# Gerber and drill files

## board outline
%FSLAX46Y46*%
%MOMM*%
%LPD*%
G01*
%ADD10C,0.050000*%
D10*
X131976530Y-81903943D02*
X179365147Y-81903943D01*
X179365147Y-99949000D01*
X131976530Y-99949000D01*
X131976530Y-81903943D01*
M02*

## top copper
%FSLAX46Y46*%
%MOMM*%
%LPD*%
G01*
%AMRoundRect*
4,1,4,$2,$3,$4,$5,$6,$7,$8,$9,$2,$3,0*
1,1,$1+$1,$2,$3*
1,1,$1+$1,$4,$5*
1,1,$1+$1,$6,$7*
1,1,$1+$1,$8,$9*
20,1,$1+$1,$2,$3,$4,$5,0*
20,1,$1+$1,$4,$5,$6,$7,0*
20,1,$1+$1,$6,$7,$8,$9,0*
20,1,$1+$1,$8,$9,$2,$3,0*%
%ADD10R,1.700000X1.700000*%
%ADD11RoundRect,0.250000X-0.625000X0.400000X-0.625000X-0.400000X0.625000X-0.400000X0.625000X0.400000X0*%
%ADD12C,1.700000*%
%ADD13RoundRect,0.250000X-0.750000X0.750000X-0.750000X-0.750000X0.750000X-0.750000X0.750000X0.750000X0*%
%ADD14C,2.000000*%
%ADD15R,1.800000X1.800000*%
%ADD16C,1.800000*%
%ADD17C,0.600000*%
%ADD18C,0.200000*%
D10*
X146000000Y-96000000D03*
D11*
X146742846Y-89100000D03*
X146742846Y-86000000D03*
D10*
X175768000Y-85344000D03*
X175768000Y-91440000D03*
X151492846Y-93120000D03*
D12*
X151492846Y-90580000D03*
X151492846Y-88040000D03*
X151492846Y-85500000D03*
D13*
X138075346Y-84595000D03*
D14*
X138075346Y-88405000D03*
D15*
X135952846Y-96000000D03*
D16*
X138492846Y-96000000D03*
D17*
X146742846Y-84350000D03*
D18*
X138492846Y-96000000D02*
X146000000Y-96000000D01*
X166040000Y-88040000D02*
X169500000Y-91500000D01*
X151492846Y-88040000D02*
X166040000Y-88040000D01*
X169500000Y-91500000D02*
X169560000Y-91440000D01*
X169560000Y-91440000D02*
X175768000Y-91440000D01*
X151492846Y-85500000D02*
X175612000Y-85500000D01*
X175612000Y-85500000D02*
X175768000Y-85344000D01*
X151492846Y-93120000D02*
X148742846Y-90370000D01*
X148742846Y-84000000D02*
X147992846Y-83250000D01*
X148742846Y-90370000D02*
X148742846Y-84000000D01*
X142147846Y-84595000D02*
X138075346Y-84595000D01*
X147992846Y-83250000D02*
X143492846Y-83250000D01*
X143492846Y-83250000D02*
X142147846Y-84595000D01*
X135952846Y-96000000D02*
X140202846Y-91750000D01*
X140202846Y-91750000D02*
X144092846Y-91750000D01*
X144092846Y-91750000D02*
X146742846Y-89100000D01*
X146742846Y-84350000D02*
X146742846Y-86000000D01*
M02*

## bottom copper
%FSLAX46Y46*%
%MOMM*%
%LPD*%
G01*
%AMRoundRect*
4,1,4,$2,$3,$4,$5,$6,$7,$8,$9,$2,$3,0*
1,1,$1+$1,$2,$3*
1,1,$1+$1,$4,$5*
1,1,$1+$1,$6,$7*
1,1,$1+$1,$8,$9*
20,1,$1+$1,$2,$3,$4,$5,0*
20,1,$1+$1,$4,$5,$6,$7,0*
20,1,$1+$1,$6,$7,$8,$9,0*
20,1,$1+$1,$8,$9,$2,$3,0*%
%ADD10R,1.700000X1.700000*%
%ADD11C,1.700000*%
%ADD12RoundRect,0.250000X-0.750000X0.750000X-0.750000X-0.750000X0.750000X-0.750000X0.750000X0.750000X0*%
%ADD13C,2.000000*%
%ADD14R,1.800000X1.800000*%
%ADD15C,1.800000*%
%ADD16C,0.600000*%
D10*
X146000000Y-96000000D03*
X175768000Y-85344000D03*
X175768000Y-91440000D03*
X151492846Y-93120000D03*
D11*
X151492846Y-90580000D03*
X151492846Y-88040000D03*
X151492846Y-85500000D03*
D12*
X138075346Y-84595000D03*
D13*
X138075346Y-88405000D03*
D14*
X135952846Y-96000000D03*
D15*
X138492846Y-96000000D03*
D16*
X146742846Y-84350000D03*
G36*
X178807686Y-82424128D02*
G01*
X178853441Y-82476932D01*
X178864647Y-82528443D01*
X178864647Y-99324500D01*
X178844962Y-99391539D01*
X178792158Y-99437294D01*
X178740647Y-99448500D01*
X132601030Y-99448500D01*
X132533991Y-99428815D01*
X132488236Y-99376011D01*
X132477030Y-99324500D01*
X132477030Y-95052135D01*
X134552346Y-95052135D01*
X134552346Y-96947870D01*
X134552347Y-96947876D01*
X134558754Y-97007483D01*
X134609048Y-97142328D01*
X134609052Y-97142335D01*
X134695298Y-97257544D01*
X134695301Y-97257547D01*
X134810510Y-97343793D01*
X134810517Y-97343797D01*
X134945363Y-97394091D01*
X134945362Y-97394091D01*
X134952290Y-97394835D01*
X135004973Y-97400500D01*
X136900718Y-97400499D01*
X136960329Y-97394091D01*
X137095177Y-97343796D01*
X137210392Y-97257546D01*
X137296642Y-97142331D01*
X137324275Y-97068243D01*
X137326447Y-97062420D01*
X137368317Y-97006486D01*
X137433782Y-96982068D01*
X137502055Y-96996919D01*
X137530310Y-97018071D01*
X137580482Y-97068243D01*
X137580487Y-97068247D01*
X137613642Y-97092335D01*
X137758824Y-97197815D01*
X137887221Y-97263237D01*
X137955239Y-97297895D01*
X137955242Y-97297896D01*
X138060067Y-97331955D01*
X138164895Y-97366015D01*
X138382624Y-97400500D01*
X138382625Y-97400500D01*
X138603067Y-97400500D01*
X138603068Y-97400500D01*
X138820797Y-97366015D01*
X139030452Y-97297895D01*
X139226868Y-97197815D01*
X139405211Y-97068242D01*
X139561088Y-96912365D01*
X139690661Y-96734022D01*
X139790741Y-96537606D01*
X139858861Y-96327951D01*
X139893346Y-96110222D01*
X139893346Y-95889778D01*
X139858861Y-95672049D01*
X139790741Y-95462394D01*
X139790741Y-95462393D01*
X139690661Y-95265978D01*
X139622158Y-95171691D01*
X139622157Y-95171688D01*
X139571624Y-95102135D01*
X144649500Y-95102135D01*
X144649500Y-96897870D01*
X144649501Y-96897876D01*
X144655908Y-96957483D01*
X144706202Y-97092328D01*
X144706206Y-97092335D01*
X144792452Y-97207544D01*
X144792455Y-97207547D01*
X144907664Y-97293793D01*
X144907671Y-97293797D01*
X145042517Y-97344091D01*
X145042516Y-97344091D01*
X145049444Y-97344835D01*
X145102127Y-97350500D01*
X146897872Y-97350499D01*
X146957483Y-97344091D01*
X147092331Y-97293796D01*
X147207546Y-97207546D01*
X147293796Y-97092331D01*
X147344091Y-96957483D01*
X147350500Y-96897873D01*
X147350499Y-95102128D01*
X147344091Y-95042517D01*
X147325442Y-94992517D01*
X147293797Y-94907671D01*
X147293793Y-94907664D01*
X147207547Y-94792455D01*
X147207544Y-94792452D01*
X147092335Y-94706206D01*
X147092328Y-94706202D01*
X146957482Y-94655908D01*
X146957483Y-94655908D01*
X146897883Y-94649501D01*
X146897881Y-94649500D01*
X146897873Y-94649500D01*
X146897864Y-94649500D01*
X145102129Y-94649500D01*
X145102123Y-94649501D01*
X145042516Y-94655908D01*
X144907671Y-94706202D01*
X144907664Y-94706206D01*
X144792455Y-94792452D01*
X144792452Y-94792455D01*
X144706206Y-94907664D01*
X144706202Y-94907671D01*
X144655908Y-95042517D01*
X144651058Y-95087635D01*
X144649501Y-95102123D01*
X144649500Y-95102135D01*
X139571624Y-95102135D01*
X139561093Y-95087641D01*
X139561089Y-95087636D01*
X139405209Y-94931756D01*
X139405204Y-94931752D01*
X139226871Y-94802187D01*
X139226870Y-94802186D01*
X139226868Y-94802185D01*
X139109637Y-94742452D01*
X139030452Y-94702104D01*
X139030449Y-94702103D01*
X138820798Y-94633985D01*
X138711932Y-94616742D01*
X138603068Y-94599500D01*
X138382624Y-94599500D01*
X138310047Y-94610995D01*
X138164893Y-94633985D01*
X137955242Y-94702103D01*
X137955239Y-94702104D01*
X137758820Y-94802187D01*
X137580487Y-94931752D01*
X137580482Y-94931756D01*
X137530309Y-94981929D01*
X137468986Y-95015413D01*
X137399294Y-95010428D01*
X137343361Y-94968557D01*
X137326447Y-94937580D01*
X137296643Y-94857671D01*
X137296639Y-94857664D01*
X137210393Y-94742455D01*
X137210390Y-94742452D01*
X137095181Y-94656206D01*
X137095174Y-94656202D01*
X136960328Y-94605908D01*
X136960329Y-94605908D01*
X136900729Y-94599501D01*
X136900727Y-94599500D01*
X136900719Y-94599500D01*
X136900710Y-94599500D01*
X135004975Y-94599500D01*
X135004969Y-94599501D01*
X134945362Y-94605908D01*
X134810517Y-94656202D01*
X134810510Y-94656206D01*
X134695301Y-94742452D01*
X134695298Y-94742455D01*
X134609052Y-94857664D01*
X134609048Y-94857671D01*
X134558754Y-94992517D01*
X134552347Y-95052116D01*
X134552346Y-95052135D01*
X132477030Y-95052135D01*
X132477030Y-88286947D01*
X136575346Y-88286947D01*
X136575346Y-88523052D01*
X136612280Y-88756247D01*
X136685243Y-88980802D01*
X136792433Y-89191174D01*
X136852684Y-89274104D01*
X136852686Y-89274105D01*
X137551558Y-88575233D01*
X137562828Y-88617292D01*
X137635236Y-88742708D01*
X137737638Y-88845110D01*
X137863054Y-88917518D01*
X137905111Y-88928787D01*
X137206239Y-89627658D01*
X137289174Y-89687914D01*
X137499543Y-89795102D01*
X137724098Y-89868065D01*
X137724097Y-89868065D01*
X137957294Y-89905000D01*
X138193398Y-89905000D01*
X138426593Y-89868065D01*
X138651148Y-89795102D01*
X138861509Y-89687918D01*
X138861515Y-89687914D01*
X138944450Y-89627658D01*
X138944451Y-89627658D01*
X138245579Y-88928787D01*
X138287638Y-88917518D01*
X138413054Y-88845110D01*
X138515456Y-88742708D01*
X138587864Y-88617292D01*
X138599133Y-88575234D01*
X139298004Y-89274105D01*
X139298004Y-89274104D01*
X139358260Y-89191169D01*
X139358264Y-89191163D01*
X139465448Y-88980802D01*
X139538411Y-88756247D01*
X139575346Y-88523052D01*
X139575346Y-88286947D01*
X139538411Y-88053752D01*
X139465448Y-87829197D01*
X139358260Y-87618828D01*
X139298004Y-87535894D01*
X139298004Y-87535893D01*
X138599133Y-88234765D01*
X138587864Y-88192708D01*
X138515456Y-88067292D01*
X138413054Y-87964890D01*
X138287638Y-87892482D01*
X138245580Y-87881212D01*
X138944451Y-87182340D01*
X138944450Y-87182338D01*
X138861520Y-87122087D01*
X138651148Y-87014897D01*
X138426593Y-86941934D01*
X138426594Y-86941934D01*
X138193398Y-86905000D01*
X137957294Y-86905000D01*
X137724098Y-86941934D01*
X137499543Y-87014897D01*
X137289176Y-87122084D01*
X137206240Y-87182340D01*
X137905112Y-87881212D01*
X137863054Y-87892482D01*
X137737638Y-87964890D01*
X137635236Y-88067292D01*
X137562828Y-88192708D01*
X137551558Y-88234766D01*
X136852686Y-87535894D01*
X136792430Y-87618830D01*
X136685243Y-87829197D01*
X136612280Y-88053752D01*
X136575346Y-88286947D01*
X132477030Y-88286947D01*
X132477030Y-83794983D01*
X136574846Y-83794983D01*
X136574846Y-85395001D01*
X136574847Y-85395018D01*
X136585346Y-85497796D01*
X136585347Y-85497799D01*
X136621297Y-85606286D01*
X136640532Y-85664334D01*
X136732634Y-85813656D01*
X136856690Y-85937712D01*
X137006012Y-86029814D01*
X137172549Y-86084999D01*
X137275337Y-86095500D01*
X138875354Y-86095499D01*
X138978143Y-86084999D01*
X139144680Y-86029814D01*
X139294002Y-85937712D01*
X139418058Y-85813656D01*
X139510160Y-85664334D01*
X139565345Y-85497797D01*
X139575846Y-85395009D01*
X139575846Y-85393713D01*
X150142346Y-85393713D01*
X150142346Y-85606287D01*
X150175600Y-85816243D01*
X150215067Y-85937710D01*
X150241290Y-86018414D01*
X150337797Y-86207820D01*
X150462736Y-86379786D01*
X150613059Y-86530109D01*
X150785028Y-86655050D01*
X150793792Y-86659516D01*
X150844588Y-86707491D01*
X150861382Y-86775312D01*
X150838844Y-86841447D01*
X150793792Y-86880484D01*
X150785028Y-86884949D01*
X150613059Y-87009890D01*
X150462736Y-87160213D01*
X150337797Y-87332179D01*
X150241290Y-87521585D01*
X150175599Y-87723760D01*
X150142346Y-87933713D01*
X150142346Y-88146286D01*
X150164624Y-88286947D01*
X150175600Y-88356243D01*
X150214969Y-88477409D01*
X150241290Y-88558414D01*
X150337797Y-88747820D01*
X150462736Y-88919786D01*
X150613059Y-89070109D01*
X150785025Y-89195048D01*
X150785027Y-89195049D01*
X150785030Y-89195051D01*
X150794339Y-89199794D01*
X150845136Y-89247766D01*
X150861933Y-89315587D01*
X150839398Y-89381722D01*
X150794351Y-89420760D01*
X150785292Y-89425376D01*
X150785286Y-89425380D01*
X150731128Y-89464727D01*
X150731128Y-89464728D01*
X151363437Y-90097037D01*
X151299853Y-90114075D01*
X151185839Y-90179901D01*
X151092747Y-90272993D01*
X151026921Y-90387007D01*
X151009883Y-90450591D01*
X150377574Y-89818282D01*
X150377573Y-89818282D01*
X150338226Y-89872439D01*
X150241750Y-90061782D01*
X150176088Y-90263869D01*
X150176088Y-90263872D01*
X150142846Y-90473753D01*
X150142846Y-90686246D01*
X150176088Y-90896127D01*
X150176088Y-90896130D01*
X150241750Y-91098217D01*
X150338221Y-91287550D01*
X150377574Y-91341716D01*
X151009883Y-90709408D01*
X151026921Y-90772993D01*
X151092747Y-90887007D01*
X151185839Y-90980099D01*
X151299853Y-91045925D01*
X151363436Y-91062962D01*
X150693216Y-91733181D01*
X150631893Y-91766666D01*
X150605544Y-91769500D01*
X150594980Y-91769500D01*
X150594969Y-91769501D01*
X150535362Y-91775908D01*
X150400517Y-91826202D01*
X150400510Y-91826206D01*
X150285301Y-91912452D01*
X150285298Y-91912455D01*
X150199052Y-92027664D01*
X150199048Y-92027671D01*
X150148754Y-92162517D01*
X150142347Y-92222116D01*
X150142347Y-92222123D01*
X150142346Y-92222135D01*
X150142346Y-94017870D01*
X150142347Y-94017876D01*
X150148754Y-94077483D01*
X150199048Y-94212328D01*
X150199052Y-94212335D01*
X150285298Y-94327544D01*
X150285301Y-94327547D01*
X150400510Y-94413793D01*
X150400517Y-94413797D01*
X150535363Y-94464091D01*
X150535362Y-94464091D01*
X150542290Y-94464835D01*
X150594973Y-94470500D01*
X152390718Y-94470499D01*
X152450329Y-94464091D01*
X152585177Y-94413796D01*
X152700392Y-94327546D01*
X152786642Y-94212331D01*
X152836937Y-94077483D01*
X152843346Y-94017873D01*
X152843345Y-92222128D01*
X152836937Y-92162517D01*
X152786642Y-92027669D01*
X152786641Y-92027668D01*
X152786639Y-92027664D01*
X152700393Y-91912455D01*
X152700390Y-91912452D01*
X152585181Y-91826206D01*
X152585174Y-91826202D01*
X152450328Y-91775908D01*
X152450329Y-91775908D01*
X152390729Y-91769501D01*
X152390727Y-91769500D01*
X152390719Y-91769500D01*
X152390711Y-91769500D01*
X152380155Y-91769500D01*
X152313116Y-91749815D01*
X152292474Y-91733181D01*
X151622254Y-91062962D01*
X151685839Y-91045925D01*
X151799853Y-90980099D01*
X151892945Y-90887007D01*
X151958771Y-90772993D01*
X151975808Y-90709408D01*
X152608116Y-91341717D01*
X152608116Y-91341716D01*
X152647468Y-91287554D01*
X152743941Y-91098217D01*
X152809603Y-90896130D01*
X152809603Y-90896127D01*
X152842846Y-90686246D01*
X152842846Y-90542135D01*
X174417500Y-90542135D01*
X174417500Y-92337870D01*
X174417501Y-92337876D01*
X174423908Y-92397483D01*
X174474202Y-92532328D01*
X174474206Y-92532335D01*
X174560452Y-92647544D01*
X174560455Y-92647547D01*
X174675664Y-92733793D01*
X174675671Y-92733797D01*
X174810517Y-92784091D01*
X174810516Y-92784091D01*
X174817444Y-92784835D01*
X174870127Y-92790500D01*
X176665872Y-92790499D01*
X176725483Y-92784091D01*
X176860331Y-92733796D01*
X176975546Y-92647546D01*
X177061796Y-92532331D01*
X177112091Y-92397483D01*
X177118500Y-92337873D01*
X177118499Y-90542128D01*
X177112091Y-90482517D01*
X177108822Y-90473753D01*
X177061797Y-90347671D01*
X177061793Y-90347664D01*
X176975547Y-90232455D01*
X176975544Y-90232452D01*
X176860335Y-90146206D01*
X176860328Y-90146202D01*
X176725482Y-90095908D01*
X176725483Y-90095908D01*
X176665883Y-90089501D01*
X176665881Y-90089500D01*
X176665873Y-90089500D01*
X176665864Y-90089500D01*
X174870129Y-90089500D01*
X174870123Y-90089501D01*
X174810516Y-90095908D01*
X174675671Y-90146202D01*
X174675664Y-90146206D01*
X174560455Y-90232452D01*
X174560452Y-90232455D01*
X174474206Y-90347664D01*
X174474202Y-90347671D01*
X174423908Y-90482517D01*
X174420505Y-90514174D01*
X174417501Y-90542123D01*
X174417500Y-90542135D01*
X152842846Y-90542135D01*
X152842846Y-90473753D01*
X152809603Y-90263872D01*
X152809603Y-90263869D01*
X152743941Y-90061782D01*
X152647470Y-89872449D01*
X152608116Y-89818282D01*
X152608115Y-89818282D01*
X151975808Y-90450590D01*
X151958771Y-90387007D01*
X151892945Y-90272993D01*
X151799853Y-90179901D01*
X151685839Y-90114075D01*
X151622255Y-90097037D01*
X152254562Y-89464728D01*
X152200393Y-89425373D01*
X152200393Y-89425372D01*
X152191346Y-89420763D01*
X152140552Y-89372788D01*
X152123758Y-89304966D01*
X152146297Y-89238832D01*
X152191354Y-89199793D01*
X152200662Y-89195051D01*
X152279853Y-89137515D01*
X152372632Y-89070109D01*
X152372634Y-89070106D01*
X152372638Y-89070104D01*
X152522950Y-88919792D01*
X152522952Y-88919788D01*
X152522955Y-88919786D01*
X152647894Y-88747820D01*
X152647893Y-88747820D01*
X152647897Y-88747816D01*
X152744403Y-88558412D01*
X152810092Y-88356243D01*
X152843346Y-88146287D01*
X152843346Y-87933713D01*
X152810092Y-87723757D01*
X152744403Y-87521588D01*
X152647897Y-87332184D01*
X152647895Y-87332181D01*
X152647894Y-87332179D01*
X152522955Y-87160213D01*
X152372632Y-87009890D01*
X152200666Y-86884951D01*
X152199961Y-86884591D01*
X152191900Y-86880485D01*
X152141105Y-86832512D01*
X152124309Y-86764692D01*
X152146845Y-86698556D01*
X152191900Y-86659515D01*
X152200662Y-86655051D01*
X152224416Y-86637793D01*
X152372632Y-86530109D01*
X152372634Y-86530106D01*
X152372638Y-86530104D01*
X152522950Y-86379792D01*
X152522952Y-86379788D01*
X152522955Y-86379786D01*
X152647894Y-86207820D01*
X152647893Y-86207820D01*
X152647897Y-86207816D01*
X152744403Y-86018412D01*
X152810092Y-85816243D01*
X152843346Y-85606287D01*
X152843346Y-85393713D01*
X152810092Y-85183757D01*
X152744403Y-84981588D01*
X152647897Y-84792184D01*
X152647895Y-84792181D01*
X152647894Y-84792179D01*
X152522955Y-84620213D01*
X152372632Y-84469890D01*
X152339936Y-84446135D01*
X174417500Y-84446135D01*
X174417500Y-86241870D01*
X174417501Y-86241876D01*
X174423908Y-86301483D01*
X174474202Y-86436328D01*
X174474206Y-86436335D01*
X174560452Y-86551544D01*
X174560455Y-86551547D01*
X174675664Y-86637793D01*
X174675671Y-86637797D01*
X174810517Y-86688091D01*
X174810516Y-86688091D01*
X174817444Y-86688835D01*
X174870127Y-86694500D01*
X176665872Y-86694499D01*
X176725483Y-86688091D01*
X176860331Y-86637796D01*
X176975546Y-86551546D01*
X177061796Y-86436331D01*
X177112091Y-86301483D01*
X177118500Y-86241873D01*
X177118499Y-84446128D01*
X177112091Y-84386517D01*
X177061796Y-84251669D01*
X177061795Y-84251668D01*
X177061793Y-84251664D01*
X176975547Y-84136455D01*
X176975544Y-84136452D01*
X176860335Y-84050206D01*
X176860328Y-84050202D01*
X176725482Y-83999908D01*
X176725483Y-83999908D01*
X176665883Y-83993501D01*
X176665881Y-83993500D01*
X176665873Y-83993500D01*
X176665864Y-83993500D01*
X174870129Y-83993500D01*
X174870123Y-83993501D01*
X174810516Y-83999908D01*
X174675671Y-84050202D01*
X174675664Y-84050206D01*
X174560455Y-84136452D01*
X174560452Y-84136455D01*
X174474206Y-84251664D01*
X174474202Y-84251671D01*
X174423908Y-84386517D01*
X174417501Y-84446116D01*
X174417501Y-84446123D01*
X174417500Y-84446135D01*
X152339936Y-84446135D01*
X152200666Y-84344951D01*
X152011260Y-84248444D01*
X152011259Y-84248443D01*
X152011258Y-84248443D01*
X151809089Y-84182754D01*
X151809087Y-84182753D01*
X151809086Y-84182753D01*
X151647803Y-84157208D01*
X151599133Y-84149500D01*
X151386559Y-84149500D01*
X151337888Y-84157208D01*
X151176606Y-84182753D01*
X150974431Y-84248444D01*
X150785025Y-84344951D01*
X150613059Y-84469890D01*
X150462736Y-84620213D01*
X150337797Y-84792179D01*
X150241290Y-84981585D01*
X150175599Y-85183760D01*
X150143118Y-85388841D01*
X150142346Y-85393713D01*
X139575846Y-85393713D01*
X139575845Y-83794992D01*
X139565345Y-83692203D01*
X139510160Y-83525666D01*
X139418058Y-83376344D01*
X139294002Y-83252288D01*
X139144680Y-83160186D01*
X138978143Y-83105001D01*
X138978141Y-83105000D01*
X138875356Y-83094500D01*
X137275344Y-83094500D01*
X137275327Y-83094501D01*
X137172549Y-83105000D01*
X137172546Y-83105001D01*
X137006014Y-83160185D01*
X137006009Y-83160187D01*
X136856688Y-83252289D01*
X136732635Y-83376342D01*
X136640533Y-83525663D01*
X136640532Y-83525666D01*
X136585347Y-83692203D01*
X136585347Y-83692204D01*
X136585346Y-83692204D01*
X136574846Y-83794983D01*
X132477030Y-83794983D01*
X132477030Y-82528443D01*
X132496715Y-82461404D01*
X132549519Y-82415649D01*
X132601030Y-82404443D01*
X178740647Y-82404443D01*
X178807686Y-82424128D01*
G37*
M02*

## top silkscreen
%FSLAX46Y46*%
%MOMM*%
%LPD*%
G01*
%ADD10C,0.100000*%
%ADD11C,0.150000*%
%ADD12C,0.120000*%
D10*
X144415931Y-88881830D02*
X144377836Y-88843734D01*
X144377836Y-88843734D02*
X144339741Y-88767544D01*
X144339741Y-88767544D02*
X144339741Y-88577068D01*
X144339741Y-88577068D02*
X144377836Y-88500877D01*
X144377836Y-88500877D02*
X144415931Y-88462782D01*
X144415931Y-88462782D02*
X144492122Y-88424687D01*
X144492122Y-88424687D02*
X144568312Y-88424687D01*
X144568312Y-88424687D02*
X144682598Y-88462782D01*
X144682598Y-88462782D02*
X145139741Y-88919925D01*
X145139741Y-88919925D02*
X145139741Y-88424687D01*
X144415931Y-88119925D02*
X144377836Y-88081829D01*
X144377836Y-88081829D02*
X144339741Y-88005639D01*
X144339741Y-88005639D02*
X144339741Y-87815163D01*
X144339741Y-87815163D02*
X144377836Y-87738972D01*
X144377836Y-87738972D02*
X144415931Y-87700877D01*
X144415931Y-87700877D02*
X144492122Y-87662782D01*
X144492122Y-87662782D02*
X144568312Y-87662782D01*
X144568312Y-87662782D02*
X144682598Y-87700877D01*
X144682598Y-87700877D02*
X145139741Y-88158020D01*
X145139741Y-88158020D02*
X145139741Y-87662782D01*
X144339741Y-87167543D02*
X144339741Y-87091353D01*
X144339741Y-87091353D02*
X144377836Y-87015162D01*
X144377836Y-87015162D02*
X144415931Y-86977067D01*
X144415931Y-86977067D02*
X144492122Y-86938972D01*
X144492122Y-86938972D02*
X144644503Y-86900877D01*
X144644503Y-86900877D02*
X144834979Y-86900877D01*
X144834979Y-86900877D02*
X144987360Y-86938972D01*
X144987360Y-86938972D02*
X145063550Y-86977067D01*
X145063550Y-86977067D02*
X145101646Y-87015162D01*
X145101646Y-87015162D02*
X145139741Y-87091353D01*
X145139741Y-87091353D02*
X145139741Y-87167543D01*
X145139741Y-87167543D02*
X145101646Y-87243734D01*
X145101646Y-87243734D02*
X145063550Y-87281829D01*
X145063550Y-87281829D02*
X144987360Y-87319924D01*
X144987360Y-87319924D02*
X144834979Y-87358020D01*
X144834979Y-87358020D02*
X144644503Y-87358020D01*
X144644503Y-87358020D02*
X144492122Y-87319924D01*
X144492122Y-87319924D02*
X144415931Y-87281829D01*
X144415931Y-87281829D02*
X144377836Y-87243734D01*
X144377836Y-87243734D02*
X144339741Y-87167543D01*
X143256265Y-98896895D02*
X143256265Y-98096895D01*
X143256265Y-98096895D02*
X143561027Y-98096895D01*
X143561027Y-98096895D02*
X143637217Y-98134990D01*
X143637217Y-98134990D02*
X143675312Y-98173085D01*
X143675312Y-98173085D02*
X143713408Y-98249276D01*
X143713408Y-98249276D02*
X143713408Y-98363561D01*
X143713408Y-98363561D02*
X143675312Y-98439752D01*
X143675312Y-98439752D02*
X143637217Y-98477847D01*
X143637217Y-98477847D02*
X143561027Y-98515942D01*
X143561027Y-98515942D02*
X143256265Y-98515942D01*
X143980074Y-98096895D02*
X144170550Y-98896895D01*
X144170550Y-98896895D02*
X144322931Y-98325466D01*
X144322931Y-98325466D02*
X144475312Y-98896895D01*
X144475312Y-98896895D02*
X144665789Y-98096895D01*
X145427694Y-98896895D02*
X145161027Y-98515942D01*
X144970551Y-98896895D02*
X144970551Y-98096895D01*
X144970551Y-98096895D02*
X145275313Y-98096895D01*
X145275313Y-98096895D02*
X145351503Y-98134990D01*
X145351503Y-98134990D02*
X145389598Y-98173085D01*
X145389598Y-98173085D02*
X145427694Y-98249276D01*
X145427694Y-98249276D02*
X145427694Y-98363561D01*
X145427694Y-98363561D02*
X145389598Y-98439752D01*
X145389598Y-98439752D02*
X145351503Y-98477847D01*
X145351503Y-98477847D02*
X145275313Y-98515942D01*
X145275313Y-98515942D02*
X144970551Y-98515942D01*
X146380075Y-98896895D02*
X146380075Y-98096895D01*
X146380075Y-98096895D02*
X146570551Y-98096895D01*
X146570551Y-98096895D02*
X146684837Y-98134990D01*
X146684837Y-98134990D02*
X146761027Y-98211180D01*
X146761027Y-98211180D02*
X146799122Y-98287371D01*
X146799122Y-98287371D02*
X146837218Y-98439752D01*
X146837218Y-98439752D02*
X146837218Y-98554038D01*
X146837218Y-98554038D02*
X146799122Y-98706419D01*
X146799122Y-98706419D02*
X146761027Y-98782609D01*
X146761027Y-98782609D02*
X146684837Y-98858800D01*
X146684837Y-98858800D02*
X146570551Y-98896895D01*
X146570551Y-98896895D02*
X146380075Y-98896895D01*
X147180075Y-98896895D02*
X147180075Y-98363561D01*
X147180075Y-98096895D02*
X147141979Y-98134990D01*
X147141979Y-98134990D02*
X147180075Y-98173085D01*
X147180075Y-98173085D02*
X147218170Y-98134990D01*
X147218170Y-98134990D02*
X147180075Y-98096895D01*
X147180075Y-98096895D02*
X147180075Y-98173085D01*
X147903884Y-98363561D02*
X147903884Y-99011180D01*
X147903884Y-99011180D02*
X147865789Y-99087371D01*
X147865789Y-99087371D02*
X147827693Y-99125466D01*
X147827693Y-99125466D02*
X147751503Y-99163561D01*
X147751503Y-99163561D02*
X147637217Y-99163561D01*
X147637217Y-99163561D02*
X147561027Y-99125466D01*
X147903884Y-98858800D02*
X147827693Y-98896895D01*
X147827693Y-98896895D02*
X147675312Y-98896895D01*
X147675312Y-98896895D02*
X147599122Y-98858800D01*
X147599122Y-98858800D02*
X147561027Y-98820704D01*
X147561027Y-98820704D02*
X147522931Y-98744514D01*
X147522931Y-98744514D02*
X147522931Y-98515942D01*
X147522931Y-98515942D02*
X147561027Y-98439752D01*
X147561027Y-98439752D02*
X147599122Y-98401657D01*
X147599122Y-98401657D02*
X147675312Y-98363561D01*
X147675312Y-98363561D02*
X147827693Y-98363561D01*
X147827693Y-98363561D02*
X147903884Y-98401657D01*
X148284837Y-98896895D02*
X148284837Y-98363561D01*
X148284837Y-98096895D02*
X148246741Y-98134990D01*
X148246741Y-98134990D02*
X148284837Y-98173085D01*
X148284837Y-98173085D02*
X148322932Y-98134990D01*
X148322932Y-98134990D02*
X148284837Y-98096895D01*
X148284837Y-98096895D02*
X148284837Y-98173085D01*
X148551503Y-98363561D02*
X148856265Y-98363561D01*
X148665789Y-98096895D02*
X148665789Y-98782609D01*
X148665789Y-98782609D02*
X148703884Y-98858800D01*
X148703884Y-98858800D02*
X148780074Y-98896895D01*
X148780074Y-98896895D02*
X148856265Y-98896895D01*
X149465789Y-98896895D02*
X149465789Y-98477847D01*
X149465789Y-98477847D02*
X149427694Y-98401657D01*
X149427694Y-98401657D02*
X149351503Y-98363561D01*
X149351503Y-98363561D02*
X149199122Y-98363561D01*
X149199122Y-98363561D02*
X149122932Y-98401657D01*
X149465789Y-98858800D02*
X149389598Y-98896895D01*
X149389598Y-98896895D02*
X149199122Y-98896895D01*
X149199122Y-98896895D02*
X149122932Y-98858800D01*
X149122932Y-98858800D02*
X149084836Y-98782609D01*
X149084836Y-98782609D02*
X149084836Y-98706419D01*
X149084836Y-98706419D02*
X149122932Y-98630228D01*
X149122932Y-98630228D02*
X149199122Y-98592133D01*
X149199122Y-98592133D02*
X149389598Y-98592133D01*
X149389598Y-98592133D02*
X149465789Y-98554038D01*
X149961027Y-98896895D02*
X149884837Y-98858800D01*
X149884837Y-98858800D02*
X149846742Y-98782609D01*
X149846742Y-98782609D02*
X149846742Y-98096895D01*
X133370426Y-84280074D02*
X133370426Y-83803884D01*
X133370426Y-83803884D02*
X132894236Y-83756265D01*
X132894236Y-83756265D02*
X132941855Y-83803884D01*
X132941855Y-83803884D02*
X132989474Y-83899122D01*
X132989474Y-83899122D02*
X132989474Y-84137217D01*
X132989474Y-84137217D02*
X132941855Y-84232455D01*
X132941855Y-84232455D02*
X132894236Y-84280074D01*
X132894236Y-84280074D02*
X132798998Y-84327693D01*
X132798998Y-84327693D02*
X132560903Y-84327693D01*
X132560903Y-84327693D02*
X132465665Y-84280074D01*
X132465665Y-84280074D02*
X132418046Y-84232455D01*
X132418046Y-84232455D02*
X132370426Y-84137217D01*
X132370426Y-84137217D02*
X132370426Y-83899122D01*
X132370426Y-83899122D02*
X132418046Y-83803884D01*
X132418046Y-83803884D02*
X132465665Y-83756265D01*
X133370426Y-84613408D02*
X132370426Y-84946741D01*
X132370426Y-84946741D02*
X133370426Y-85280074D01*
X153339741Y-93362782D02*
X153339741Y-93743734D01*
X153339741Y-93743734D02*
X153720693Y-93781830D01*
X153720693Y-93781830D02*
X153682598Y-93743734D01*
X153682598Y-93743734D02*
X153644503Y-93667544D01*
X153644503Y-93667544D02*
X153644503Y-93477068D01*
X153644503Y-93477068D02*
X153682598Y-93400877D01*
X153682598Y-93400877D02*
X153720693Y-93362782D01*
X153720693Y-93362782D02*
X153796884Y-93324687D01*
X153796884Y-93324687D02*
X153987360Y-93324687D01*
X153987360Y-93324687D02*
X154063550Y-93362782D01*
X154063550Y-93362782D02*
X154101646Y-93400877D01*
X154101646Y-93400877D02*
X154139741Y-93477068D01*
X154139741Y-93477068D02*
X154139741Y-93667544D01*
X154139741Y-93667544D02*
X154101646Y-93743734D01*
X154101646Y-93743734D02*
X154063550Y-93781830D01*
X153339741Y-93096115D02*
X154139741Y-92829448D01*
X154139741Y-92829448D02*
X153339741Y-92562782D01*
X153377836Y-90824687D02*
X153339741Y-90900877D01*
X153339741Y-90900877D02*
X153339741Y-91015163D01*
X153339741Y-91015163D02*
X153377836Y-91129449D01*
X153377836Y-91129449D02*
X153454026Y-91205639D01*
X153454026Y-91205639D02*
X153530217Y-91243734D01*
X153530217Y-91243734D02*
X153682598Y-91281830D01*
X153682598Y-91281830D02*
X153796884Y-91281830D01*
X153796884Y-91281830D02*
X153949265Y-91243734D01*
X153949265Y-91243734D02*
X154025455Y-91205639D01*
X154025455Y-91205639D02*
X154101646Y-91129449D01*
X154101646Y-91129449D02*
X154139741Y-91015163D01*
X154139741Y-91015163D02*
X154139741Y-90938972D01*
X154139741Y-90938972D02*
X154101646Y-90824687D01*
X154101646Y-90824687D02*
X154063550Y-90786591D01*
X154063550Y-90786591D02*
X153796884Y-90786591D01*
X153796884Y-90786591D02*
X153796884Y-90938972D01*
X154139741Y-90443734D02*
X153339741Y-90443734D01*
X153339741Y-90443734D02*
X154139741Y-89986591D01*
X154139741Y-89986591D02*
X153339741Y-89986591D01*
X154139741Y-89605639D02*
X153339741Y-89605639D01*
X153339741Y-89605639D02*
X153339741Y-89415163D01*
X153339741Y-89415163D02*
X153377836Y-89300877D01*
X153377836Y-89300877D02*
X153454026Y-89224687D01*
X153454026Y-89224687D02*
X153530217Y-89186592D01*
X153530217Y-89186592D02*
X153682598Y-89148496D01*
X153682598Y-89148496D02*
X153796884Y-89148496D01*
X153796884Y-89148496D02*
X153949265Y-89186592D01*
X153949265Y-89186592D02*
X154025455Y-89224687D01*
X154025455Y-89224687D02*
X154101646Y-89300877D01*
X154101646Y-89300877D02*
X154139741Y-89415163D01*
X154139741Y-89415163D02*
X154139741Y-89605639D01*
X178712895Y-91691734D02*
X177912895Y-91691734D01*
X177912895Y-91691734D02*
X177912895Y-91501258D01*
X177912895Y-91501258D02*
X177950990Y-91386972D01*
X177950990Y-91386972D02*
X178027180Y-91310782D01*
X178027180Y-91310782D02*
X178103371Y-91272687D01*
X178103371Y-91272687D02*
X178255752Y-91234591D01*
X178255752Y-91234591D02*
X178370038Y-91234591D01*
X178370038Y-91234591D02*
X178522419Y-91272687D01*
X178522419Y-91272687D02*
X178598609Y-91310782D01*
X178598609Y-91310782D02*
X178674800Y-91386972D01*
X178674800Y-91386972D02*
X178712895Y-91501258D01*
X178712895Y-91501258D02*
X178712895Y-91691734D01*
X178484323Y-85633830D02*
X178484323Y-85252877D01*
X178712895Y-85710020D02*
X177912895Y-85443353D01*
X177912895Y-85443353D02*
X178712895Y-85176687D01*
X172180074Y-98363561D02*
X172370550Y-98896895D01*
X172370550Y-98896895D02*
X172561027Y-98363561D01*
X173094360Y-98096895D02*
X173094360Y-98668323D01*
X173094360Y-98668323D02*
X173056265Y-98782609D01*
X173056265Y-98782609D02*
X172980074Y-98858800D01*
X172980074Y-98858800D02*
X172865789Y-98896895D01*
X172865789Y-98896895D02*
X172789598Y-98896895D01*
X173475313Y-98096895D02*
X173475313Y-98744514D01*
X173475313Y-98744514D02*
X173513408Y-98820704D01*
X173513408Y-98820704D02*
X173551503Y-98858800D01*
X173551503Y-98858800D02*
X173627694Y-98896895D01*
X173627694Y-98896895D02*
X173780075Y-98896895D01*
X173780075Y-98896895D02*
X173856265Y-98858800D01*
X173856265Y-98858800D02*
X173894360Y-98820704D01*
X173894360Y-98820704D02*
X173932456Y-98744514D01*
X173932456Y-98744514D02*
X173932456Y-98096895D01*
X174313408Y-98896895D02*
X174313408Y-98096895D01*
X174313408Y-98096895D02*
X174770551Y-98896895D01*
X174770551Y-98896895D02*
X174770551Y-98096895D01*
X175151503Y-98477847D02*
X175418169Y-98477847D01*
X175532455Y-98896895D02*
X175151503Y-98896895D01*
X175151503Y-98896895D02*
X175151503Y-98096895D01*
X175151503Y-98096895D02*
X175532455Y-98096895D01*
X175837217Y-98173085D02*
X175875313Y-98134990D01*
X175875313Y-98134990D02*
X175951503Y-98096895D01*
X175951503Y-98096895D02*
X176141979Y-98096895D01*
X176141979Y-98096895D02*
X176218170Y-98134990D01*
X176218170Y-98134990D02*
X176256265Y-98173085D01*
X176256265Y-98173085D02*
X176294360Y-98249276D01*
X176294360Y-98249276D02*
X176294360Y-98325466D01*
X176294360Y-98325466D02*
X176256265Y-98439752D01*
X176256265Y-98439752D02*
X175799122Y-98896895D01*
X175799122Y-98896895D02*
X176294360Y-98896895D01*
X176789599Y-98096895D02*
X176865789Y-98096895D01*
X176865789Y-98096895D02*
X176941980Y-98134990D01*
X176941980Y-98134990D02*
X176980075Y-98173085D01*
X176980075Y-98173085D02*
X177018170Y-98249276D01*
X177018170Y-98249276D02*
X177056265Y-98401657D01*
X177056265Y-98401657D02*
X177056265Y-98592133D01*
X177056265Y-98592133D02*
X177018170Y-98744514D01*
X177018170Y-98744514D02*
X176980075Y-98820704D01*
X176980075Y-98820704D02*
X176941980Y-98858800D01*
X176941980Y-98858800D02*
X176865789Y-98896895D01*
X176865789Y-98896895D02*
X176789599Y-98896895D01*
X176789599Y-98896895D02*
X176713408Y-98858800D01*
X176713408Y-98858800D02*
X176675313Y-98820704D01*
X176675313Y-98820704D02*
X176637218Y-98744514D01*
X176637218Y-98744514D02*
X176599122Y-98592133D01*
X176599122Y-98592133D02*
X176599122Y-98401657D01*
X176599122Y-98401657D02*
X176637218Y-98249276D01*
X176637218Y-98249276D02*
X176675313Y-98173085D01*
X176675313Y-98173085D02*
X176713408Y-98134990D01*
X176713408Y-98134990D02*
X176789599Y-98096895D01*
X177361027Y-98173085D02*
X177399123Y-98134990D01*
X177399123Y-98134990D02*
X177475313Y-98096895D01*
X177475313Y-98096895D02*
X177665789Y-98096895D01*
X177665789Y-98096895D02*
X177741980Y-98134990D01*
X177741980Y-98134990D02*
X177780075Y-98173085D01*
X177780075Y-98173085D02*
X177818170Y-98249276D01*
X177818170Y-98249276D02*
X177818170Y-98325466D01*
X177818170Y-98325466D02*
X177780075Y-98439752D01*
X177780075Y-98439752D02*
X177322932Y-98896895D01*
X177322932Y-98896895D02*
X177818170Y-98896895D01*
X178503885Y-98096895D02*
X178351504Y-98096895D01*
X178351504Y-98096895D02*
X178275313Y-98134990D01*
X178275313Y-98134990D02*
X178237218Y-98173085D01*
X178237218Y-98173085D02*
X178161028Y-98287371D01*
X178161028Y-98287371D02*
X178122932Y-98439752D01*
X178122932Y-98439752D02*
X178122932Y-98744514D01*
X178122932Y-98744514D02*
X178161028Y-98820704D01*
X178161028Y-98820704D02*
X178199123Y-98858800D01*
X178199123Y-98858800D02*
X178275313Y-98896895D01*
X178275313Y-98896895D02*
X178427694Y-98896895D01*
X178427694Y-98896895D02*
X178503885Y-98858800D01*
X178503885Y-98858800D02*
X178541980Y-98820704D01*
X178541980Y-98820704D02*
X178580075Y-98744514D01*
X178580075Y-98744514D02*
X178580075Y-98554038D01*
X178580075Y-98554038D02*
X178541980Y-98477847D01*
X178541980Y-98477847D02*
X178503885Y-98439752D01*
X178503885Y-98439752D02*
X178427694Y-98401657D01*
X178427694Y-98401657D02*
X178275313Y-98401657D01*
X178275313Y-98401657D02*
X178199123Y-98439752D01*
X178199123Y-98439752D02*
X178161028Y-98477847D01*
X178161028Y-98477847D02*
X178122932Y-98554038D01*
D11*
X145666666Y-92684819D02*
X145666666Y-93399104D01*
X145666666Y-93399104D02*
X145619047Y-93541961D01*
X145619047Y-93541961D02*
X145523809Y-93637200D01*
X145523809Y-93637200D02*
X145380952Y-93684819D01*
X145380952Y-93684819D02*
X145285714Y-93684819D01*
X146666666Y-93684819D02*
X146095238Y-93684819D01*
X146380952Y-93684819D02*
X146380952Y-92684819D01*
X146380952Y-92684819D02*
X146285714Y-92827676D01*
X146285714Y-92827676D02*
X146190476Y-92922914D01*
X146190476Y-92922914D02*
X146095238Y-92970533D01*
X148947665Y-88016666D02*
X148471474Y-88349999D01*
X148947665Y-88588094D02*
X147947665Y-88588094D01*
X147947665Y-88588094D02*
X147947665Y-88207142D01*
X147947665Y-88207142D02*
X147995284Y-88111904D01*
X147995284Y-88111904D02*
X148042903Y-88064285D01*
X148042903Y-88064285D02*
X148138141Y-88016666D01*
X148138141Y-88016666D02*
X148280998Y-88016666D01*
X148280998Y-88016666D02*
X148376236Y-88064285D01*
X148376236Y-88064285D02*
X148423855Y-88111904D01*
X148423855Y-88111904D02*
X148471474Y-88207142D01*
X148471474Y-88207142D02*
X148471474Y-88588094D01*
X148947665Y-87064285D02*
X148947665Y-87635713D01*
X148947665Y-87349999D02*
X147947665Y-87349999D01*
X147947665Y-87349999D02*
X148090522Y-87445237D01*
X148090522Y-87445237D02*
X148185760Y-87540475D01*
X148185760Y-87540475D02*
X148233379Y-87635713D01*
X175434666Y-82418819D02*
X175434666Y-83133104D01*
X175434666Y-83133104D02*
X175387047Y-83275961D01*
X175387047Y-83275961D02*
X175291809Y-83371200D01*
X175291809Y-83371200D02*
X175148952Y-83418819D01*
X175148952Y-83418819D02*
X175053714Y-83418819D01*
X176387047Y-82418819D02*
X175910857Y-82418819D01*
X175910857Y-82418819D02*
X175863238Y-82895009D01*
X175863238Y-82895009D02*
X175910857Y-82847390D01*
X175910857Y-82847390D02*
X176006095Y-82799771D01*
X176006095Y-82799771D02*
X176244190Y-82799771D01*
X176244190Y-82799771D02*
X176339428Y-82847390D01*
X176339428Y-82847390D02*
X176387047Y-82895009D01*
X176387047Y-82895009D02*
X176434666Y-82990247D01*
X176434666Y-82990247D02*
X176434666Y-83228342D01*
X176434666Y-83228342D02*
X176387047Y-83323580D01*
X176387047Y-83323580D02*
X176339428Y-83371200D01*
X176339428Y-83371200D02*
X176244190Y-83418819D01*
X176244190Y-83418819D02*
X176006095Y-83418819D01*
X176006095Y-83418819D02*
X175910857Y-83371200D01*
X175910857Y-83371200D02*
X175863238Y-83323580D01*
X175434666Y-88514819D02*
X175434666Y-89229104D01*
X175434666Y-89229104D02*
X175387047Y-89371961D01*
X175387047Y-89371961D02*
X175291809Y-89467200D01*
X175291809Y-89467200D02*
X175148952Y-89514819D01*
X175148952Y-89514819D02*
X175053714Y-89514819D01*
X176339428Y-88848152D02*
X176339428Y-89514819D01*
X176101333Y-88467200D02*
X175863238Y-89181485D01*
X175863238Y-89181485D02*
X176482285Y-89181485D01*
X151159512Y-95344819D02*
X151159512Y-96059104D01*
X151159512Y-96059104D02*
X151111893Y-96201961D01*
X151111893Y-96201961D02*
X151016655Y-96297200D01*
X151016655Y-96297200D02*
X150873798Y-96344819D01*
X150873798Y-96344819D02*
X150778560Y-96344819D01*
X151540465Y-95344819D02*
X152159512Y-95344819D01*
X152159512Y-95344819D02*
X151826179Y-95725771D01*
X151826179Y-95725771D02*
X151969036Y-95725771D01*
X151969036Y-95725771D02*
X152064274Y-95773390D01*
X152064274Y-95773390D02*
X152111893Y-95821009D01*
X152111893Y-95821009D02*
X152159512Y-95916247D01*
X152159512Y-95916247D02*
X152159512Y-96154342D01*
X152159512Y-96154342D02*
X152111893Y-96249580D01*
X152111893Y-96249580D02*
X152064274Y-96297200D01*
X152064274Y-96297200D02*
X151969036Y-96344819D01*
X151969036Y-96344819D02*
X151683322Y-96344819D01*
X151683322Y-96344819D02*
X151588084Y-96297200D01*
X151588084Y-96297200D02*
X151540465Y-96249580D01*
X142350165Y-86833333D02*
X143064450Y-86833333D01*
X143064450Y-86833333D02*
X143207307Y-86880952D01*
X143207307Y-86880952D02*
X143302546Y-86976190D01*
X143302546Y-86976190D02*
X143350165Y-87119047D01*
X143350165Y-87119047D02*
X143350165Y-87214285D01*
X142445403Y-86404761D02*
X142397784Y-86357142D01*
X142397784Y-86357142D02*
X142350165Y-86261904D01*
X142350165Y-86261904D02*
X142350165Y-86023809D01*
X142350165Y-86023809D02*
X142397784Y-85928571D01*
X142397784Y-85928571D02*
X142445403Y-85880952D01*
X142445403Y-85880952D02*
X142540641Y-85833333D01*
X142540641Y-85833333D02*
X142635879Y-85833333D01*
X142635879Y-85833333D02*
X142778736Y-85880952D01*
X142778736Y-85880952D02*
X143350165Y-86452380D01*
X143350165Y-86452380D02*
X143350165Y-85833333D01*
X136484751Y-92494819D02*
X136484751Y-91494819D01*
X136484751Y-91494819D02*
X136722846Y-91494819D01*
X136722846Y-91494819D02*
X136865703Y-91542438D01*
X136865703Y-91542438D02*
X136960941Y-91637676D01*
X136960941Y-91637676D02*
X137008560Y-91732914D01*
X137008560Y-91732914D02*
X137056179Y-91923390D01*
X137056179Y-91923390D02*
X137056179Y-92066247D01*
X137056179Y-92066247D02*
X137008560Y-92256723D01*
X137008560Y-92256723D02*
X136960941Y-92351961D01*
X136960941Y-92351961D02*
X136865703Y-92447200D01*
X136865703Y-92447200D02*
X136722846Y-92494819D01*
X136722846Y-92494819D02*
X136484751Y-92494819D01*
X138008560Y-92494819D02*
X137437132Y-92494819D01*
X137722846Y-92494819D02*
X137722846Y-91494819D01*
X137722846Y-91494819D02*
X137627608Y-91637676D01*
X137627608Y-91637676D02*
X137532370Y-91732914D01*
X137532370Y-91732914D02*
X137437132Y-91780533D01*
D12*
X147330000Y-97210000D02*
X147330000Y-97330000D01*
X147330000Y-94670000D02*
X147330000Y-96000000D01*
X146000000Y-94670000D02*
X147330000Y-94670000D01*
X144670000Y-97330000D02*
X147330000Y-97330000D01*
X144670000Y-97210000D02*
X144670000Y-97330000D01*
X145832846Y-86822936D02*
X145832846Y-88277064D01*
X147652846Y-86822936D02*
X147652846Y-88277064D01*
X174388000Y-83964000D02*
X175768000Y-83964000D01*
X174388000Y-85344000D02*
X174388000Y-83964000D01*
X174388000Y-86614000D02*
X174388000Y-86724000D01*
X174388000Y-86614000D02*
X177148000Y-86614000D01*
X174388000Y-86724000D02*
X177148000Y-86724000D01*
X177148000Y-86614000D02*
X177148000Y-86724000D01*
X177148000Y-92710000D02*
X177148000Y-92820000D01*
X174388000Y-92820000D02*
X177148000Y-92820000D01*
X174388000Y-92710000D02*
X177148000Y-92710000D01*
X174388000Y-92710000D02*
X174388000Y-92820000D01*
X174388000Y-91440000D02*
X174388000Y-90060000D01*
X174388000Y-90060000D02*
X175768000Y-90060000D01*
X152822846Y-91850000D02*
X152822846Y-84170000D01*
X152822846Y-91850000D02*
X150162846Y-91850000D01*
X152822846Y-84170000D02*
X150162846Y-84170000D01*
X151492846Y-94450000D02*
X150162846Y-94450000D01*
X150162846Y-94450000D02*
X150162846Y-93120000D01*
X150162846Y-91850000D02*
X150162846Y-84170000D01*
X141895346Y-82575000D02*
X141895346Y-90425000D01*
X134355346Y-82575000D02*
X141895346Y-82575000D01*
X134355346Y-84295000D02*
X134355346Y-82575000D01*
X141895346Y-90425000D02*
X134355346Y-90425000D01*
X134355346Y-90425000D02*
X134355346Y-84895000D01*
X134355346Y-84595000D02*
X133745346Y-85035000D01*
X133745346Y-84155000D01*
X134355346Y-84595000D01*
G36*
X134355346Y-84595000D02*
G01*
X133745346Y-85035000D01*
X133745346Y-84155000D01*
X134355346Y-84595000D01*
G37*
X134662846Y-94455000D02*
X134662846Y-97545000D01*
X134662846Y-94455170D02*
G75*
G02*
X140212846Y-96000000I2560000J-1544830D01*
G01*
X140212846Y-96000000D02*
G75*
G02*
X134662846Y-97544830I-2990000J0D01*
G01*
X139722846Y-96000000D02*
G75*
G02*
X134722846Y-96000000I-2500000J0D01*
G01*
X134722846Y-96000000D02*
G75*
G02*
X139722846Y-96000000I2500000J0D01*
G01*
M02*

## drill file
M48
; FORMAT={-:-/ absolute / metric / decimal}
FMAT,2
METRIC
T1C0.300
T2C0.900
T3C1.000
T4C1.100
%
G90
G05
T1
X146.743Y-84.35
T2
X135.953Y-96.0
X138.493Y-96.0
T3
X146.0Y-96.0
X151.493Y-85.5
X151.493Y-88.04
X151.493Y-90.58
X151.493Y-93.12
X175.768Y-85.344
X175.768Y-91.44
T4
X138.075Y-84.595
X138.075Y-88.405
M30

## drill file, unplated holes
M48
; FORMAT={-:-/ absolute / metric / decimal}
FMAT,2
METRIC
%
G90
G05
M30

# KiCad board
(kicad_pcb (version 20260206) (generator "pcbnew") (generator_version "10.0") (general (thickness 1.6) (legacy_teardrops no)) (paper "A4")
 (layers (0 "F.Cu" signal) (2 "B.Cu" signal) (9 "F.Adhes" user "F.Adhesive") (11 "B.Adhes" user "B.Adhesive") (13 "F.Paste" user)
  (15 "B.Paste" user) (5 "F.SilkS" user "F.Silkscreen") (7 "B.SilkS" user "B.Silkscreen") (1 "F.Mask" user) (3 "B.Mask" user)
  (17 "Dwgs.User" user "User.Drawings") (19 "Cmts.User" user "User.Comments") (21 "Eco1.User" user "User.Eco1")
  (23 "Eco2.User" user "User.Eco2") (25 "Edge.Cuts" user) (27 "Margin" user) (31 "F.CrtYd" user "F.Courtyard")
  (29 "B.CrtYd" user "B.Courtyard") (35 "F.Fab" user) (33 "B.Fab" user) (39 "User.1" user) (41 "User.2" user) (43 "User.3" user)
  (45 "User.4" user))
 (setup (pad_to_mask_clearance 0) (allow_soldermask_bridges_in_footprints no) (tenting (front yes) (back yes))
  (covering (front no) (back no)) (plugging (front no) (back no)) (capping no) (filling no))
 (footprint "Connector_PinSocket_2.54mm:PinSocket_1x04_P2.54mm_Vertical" (layer "F.Cu") (at 151.492846 93.12 180)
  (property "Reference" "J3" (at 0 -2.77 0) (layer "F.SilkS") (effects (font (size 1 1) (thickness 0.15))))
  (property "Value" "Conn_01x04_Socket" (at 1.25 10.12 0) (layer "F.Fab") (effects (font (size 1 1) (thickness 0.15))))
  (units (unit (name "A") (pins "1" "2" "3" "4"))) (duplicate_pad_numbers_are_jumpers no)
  (fp_line (start 1.33 1.27) (end 1.33 8.95) (stroke (width 0.12) (type solid)) (layer "F.SilkS"))
  (fp_line (start 1.33 -1.33) (end 1.33 0) (stroke (width 0.12) (type solid)) (layer "F.SilkS"))
  (fp_line (start 0 -1.33) (end 1.33 -1.33) (stroke (width 0.12) (type solid)) (layer "F.SilkS"))
  (fp_line (start -1.33 8.95) (end 1.33 8.95) (stroke (width 0.12) (type solid)) (layer "F.SilkS"))
  (fp_line (start -1.33 1.27) (end 1.33 1.27) (stroke (width 0.12) (type solid)) (layer "F.SilkS"))
  (fp_line (start -1.33 1.27) (end -1.33 8.95) (stroke (width 0.12) (type solid)) (layer "F.SilkS"))
  (pad "1" thru_hole rect (at 0 0 180) (size 1.7 1.7) (drill 1) (layers "*.Cu" "*.Mask") (remove_unused_layers no) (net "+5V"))
  (pad "2" thru_hole circle (at 0 2.54 180) (size 1.7 1.7) (drill 1) (layers "*.Cu" "*.Mask") (remove_unused_layers no) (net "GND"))
  (pad "3" thru_hole circle (at 0 5.08 180) (size 1.7 1.7) (drill 1) (layers "*.Cu" "*.Mask") (remove_unused_layers no) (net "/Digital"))
  (pad "4" thru_hole circle (at 0 7.62 180) (size 1.7 1.7) (drill 1) (layers "*.Cu" "*.Mask") (remove_unused_layers no) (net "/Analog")))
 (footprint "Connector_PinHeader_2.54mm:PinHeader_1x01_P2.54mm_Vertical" (layer "F.Cu") (at 175.768 85.344)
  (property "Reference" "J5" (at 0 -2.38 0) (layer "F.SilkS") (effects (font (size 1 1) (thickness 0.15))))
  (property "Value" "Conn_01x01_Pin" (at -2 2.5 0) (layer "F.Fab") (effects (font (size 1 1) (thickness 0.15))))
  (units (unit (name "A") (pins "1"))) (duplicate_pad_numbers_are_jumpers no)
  (fp_line (start -1.38 -1.38) (end 0 -1.38) (stroke (width 0.12) (type solid)) (layer "F.SilkS"))
  (fp_line (start -1.38 0) (end -1.38 -1.38) (stroke (width 0.12) (type solid)) (layer "F.SilkS"))
  (fp_line (start -1.38 1.27) (end -1.38 1.38) (stroke (width 0.12) (type solid)) (layer "F.SilkS"))
  (fp_line (start -1.38 1.27) (end 1.38 1.27) (stroke (width 0.12) (type solid)) (layer "F.SilkS"))
  (fp_line (start -1.38 1.38) (end 1.38 1.38) (stroke (width 0.12) (type solid)) (layer "F.SilkS"))
  (fp_line (start 1.38 1.27) (end 1.38 1.38) (stroke (width 0.12) (type solid)) (layer "F.SilkS"))
  (pad "1" thru_hole rect (at 0 0) (size 1.7 1.7) (drill 1) (layers "*.Cu" "*.Mask") (remove_unused_layers no) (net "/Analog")))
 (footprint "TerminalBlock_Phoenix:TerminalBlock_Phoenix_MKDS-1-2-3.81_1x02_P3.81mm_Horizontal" (layer "F.Cu") (at 138.075346 84.595 -90)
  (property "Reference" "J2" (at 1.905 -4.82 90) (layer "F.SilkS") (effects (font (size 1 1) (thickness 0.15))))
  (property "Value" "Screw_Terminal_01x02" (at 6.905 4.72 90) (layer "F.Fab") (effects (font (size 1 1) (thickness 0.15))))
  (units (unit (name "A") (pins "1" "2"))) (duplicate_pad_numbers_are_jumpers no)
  (fp_line (start -2.02 3.72) (end -2.02 -3.82) (stroke (width 0.12) (type solid)) (layer "F.SilkS"))
  (fp_line (start -0.3 3.72) (end -2.02 3.72) (stroke (width 0.12) (type solid)) (layer "F.SilkS"))
  (fp_line (start 5.83 3.72) (end 0.3 3.72) (stroke (width 0.12) (type solid)) (layer "F.SilkS"))
  (fp_line (start -2.02 -3.82) (end 5.83 -3.82) (stroke (width 0.12) (type solid)) (layer "F.SilkS"))
  (fp_line (start 5.83 -3.82) (end 5.83 3.72) (stroke (width 0.12) (type solid)) (layer "F.SilkS"))
  (fp_poly (pts (xy 0 3.72) (xy 0.44 4.33) (xy -0.44 4.33)) (stroke (width 0.12) (type solid)) (fill yes) (layer "F.SilkS"))
  (pad "1" thru_hole roundrect (at 0 0 270) (size 2 2) (drill 1.1) (layers "*.Cu" "*.Mask") (remove_unused_layers no)
   (roundrect_rratio 0.125) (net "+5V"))
  (pad "2" thru_hole circle (at 3.81 0 270) (size 2 2) (drill 1.1) (layers "*.Cu" "*.Mask") (remove_unused_layers no) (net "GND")))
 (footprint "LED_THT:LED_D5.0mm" (layer "F.Cu") (at 135.952846 96)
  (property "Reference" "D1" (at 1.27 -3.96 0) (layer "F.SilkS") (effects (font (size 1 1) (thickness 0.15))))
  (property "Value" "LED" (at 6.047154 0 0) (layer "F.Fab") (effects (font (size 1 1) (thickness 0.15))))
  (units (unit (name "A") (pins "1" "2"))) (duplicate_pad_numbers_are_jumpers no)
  (fp_line (start -1.29 -1.545) (end -1.29 1.545) (stroke (width 0.12) (type solid)) (layer "F.SilkS"))
  (fp_arc (start -1.29 -1.54483) (mid 2.071779 -2.880495) (end 4.26 0) (stroke (width 0.12) (type solid)) (layer "F.SilkS"))
  (fp_arc (start 4.26 0) (mid 2.071779 2.880495) (end -1.29 1.54483) (stroke (width 0.12) (type solid)) (layer "F.SilkS"))
  (fp_circle (center 1.27 0) (end 3.77 0) (stroke (width 0.12) (type solid)) (fill no) (layer "F.SilkS"))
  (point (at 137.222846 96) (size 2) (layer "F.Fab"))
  (pad "1" thru_hole rect (at 0 0) (size 1.8 1.8) (drill 0.9) (layers "*.Cu" "*.Mask") (remove_unused_layers no) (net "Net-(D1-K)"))
  (pad "2" thru_hole circle (at 2.54 0) (size 1.8 1.8) (drill 0.9) (layers "*.Cu" "*.Mask") (remove_unused_layers no) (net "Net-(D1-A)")))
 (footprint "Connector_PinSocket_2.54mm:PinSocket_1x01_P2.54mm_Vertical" (layer "F.Cu") (at 146 96)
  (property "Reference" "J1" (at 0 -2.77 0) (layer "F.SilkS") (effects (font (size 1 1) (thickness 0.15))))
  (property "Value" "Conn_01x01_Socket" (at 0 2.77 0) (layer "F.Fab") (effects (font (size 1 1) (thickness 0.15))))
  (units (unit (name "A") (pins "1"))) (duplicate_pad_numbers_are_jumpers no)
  (fp_line (start -1.33 1.21) (end -1.33 1.33) (stroke (width 0.12) (type solid)) (layer "F.SilkS"))
  (fp_line (start -1.33 1.33) (end 1.33 1.33) (stroke (width 0.12) (type solid)) (layer "F.SilkS"))
  (fp_line (start 0 -1.33) (end 1.33 -1.33) (stroke (width 0.12) (type solid)) (layer "F.SilkS"))
  (fp_line (start 1.33 -1.33) (end 1.33 0) (stroke (width 0.12) (type solid)) (layer "F.SilkS"))
  (fp_line (start 1.33 1.21) (end 1.33 1.33) (stroke (width 0.12) (type solid)) (layer "F.SilkS"))
  (pad "1" thru_hole rect (at 0 0) (size 1.7 1.7) (drill 1) (layers "*.Cu" "*.Mask") (remove_unused_layers no) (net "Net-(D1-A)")))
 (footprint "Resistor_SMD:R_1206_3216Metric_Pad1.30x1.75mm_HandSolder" (layer "F.Cu") (at 146.742846 87.55 -90)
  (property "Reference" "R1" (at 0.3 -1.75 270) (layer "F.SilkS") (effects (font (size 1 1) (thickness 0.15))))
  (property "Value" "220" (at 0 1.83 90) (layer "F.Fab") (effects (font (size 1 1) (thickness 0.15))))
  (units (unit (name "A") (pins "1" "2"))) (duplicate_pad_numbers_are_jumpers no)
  (fp_line (start -0.727064 0.91) (end 0.727064 0.91) (stroke (width 0.12) (type solid)) (layer "F.SilkS"))
  (fp_line (start -0.727064 -0.91) (end 0.727064 -0.91) (stroke (width 0.12) (type solid)) (layer "F.SilkS"))
  (pad "1" smd roundrect (at -1.55 0 270) (size 1.3 1.75) (layers "F.Cu" "F.Mask" "F.Paste") (roundrect_rratio 0.192308) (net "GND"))
  (pad "2" smd roundrect (at 1.55 0 270) (size 1.3 1.75) (layers "F.Cu" "F.Mask" "F.Paste") (roundrect_rratio 0.192308) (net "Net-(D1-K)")))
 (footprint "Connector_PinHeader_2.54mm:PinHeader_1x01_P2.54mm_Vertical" (layer "F.Cu") (at 175.768 91.44)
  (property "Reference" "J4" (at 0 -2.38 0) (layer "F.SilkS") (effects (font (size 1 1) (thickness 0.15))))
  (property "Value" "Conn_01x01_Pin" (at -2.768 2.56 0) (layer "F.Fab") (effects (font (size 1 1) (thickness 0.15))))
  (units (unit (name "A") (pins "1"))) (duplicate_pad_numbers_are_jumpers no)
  (fp_line (start -1.38 -1.38) (end 0 -1.38) (stroke (width 0.12) (type solid)) (layer "F.SilkS"))
  (fp_line (start -1.38 0) (end -1.38 -1.38) (stroke (width 0.12) (type solid)) (layer "F.SilkS"))
  (fp_line (start -1.38 1.27) (end -1.38 1.38) (stroke (width 0.12) (type solid)) (layer "F.SilkS"))
  (fp_line (start -1.38 1.27) (end 1.38 1.27) (stroke (width 0.12) (type solid)) (layer "F.SilkS"))
  (fp_line (start -1.38 1.38) (end 1.38 1.38) (stroke (width 0.12) (type solid)) (layer "F.SilkS"))
  (fp_line (start 1.38 1.27) (end 1.38 1.38) (stroke (width 0.12) (type solid)) (layer "F.SilkS"))
  (pad "1" thru_hole rect (at 0 0) (size 1.7 1.7) (drill 1) (layers "*.Cu" "*.Mask") (remove_unused_layers no) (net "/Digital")))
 (gr_rect (start 131.97653 81.903943) (end 179.365147 99.949) (stroke (width 0.05) (type default)) (fill no) (layer "Edge.Cuts"))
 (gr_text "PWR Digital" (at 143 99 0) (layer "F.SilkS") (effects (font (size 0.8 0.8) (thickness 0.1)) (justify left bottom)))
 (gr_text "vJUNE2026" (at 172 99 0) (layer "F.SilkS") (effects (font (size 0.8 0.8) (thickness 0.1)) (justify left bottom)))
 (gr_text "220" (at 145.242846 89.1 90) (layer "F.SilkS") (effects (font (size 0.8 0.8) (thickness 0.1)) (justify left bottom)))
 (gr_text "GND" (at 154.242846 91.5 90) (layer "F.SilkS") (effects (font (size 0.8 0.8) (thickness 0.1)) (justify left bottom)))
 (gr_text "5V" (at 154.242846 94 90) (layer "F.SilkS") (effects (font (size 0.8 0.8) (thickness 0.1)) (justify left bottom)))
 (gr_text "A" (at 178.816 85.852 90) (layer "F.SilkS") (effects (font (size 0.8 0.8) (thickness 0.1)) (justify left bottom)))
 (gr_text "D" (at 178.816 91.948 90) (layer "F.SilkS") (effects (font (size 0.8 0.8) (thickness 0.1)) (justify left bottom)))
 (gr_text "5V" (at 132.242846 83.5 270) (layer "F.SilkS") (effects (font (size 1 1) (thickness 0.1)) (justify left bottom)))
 (segment (start 147.992846 83.25) (end 143.492846 83.25) (width 0.2) (layer "F.Cu") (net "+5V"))
 (segment (start 143.492846 83.25) (end 142.147846 84.595) (width 0.2) (layer "F.Cu") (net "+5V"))
 (segment (start 148.742846 90.37) (end 148.742846 84) (width 0.2) (layer "F.Cu") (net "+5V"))
 (segment (start 151.492846 93.12) (end 148.742846 90.37) (width 0.2) (layer "F.Cu") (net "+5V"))
 (segment (start 142.147846 84.595) (end 138.075346 84.595) (width 0.2) (layer "F.Cu") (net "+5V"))
 (segment (start 148.742846 84) (end 147.992846 83.25) (width 0.2) (layer "F.Cu") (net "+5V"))
 (segment (start 146.742846 84.35) (end 146.742846 86) (width 0.2) (layer "F.Cu") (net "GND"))
 (via (at 146.742846 84.35) (size 0.6) (drill 0.3) (layers "F.Cu" "B.Cu") (free yes) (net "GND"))
 (segment (start 166.04 88.04) (end 169.5 91.5) (width 0.2) (layer "F.Cu") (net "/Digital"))
 (segment (start 169.56 91.44) (end 175.768 91.44) (width 0.2) (layer "F.Cu") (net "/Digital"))
 (segment (start 151.492846 88.04) (end 166.04 88.04) (width 0.2) (layer "F.Cu") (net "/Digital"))
 (segment (start 169.5 91.5) (end 169.56 91.44) (width 0.2) (layer "F.Cu") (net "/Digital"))
 (segment (start 175.612 85.5) (end 175.768 85.344) (width 0.2) (layer "F.Cu") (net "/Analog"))
 (segment (start 151.492846 85.5) (end 175.612 85.5) (width 0.2) (layer "F.Cu") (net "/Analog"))
 (segment (start 140.202846 91.75) (end 144.092846 91.75) (width 0.2) (layer "F.Cu") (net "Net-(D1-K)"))
 (segment (start 144.092846 91.75) (end 146.742846 89.1) (width 0.2) (layer "F.Cu") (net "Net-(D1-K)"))
 (segment (start 135.952846 96) (end 140.202846 91.75) (width 0.2) (layer "F.Cu") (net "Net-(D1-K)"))
 (segment (start 138.492846 96) (end 146 96) (width 0.2) (layer "F.Cu") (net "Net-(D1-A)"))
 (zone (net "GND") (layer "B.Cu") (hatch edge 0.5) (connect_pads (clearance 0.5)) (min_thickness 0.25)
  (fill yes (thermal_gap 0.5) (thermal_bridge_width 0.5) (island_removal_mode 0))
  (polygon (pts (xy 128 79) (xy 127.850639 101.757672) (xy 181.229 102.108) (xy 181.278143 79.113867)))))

